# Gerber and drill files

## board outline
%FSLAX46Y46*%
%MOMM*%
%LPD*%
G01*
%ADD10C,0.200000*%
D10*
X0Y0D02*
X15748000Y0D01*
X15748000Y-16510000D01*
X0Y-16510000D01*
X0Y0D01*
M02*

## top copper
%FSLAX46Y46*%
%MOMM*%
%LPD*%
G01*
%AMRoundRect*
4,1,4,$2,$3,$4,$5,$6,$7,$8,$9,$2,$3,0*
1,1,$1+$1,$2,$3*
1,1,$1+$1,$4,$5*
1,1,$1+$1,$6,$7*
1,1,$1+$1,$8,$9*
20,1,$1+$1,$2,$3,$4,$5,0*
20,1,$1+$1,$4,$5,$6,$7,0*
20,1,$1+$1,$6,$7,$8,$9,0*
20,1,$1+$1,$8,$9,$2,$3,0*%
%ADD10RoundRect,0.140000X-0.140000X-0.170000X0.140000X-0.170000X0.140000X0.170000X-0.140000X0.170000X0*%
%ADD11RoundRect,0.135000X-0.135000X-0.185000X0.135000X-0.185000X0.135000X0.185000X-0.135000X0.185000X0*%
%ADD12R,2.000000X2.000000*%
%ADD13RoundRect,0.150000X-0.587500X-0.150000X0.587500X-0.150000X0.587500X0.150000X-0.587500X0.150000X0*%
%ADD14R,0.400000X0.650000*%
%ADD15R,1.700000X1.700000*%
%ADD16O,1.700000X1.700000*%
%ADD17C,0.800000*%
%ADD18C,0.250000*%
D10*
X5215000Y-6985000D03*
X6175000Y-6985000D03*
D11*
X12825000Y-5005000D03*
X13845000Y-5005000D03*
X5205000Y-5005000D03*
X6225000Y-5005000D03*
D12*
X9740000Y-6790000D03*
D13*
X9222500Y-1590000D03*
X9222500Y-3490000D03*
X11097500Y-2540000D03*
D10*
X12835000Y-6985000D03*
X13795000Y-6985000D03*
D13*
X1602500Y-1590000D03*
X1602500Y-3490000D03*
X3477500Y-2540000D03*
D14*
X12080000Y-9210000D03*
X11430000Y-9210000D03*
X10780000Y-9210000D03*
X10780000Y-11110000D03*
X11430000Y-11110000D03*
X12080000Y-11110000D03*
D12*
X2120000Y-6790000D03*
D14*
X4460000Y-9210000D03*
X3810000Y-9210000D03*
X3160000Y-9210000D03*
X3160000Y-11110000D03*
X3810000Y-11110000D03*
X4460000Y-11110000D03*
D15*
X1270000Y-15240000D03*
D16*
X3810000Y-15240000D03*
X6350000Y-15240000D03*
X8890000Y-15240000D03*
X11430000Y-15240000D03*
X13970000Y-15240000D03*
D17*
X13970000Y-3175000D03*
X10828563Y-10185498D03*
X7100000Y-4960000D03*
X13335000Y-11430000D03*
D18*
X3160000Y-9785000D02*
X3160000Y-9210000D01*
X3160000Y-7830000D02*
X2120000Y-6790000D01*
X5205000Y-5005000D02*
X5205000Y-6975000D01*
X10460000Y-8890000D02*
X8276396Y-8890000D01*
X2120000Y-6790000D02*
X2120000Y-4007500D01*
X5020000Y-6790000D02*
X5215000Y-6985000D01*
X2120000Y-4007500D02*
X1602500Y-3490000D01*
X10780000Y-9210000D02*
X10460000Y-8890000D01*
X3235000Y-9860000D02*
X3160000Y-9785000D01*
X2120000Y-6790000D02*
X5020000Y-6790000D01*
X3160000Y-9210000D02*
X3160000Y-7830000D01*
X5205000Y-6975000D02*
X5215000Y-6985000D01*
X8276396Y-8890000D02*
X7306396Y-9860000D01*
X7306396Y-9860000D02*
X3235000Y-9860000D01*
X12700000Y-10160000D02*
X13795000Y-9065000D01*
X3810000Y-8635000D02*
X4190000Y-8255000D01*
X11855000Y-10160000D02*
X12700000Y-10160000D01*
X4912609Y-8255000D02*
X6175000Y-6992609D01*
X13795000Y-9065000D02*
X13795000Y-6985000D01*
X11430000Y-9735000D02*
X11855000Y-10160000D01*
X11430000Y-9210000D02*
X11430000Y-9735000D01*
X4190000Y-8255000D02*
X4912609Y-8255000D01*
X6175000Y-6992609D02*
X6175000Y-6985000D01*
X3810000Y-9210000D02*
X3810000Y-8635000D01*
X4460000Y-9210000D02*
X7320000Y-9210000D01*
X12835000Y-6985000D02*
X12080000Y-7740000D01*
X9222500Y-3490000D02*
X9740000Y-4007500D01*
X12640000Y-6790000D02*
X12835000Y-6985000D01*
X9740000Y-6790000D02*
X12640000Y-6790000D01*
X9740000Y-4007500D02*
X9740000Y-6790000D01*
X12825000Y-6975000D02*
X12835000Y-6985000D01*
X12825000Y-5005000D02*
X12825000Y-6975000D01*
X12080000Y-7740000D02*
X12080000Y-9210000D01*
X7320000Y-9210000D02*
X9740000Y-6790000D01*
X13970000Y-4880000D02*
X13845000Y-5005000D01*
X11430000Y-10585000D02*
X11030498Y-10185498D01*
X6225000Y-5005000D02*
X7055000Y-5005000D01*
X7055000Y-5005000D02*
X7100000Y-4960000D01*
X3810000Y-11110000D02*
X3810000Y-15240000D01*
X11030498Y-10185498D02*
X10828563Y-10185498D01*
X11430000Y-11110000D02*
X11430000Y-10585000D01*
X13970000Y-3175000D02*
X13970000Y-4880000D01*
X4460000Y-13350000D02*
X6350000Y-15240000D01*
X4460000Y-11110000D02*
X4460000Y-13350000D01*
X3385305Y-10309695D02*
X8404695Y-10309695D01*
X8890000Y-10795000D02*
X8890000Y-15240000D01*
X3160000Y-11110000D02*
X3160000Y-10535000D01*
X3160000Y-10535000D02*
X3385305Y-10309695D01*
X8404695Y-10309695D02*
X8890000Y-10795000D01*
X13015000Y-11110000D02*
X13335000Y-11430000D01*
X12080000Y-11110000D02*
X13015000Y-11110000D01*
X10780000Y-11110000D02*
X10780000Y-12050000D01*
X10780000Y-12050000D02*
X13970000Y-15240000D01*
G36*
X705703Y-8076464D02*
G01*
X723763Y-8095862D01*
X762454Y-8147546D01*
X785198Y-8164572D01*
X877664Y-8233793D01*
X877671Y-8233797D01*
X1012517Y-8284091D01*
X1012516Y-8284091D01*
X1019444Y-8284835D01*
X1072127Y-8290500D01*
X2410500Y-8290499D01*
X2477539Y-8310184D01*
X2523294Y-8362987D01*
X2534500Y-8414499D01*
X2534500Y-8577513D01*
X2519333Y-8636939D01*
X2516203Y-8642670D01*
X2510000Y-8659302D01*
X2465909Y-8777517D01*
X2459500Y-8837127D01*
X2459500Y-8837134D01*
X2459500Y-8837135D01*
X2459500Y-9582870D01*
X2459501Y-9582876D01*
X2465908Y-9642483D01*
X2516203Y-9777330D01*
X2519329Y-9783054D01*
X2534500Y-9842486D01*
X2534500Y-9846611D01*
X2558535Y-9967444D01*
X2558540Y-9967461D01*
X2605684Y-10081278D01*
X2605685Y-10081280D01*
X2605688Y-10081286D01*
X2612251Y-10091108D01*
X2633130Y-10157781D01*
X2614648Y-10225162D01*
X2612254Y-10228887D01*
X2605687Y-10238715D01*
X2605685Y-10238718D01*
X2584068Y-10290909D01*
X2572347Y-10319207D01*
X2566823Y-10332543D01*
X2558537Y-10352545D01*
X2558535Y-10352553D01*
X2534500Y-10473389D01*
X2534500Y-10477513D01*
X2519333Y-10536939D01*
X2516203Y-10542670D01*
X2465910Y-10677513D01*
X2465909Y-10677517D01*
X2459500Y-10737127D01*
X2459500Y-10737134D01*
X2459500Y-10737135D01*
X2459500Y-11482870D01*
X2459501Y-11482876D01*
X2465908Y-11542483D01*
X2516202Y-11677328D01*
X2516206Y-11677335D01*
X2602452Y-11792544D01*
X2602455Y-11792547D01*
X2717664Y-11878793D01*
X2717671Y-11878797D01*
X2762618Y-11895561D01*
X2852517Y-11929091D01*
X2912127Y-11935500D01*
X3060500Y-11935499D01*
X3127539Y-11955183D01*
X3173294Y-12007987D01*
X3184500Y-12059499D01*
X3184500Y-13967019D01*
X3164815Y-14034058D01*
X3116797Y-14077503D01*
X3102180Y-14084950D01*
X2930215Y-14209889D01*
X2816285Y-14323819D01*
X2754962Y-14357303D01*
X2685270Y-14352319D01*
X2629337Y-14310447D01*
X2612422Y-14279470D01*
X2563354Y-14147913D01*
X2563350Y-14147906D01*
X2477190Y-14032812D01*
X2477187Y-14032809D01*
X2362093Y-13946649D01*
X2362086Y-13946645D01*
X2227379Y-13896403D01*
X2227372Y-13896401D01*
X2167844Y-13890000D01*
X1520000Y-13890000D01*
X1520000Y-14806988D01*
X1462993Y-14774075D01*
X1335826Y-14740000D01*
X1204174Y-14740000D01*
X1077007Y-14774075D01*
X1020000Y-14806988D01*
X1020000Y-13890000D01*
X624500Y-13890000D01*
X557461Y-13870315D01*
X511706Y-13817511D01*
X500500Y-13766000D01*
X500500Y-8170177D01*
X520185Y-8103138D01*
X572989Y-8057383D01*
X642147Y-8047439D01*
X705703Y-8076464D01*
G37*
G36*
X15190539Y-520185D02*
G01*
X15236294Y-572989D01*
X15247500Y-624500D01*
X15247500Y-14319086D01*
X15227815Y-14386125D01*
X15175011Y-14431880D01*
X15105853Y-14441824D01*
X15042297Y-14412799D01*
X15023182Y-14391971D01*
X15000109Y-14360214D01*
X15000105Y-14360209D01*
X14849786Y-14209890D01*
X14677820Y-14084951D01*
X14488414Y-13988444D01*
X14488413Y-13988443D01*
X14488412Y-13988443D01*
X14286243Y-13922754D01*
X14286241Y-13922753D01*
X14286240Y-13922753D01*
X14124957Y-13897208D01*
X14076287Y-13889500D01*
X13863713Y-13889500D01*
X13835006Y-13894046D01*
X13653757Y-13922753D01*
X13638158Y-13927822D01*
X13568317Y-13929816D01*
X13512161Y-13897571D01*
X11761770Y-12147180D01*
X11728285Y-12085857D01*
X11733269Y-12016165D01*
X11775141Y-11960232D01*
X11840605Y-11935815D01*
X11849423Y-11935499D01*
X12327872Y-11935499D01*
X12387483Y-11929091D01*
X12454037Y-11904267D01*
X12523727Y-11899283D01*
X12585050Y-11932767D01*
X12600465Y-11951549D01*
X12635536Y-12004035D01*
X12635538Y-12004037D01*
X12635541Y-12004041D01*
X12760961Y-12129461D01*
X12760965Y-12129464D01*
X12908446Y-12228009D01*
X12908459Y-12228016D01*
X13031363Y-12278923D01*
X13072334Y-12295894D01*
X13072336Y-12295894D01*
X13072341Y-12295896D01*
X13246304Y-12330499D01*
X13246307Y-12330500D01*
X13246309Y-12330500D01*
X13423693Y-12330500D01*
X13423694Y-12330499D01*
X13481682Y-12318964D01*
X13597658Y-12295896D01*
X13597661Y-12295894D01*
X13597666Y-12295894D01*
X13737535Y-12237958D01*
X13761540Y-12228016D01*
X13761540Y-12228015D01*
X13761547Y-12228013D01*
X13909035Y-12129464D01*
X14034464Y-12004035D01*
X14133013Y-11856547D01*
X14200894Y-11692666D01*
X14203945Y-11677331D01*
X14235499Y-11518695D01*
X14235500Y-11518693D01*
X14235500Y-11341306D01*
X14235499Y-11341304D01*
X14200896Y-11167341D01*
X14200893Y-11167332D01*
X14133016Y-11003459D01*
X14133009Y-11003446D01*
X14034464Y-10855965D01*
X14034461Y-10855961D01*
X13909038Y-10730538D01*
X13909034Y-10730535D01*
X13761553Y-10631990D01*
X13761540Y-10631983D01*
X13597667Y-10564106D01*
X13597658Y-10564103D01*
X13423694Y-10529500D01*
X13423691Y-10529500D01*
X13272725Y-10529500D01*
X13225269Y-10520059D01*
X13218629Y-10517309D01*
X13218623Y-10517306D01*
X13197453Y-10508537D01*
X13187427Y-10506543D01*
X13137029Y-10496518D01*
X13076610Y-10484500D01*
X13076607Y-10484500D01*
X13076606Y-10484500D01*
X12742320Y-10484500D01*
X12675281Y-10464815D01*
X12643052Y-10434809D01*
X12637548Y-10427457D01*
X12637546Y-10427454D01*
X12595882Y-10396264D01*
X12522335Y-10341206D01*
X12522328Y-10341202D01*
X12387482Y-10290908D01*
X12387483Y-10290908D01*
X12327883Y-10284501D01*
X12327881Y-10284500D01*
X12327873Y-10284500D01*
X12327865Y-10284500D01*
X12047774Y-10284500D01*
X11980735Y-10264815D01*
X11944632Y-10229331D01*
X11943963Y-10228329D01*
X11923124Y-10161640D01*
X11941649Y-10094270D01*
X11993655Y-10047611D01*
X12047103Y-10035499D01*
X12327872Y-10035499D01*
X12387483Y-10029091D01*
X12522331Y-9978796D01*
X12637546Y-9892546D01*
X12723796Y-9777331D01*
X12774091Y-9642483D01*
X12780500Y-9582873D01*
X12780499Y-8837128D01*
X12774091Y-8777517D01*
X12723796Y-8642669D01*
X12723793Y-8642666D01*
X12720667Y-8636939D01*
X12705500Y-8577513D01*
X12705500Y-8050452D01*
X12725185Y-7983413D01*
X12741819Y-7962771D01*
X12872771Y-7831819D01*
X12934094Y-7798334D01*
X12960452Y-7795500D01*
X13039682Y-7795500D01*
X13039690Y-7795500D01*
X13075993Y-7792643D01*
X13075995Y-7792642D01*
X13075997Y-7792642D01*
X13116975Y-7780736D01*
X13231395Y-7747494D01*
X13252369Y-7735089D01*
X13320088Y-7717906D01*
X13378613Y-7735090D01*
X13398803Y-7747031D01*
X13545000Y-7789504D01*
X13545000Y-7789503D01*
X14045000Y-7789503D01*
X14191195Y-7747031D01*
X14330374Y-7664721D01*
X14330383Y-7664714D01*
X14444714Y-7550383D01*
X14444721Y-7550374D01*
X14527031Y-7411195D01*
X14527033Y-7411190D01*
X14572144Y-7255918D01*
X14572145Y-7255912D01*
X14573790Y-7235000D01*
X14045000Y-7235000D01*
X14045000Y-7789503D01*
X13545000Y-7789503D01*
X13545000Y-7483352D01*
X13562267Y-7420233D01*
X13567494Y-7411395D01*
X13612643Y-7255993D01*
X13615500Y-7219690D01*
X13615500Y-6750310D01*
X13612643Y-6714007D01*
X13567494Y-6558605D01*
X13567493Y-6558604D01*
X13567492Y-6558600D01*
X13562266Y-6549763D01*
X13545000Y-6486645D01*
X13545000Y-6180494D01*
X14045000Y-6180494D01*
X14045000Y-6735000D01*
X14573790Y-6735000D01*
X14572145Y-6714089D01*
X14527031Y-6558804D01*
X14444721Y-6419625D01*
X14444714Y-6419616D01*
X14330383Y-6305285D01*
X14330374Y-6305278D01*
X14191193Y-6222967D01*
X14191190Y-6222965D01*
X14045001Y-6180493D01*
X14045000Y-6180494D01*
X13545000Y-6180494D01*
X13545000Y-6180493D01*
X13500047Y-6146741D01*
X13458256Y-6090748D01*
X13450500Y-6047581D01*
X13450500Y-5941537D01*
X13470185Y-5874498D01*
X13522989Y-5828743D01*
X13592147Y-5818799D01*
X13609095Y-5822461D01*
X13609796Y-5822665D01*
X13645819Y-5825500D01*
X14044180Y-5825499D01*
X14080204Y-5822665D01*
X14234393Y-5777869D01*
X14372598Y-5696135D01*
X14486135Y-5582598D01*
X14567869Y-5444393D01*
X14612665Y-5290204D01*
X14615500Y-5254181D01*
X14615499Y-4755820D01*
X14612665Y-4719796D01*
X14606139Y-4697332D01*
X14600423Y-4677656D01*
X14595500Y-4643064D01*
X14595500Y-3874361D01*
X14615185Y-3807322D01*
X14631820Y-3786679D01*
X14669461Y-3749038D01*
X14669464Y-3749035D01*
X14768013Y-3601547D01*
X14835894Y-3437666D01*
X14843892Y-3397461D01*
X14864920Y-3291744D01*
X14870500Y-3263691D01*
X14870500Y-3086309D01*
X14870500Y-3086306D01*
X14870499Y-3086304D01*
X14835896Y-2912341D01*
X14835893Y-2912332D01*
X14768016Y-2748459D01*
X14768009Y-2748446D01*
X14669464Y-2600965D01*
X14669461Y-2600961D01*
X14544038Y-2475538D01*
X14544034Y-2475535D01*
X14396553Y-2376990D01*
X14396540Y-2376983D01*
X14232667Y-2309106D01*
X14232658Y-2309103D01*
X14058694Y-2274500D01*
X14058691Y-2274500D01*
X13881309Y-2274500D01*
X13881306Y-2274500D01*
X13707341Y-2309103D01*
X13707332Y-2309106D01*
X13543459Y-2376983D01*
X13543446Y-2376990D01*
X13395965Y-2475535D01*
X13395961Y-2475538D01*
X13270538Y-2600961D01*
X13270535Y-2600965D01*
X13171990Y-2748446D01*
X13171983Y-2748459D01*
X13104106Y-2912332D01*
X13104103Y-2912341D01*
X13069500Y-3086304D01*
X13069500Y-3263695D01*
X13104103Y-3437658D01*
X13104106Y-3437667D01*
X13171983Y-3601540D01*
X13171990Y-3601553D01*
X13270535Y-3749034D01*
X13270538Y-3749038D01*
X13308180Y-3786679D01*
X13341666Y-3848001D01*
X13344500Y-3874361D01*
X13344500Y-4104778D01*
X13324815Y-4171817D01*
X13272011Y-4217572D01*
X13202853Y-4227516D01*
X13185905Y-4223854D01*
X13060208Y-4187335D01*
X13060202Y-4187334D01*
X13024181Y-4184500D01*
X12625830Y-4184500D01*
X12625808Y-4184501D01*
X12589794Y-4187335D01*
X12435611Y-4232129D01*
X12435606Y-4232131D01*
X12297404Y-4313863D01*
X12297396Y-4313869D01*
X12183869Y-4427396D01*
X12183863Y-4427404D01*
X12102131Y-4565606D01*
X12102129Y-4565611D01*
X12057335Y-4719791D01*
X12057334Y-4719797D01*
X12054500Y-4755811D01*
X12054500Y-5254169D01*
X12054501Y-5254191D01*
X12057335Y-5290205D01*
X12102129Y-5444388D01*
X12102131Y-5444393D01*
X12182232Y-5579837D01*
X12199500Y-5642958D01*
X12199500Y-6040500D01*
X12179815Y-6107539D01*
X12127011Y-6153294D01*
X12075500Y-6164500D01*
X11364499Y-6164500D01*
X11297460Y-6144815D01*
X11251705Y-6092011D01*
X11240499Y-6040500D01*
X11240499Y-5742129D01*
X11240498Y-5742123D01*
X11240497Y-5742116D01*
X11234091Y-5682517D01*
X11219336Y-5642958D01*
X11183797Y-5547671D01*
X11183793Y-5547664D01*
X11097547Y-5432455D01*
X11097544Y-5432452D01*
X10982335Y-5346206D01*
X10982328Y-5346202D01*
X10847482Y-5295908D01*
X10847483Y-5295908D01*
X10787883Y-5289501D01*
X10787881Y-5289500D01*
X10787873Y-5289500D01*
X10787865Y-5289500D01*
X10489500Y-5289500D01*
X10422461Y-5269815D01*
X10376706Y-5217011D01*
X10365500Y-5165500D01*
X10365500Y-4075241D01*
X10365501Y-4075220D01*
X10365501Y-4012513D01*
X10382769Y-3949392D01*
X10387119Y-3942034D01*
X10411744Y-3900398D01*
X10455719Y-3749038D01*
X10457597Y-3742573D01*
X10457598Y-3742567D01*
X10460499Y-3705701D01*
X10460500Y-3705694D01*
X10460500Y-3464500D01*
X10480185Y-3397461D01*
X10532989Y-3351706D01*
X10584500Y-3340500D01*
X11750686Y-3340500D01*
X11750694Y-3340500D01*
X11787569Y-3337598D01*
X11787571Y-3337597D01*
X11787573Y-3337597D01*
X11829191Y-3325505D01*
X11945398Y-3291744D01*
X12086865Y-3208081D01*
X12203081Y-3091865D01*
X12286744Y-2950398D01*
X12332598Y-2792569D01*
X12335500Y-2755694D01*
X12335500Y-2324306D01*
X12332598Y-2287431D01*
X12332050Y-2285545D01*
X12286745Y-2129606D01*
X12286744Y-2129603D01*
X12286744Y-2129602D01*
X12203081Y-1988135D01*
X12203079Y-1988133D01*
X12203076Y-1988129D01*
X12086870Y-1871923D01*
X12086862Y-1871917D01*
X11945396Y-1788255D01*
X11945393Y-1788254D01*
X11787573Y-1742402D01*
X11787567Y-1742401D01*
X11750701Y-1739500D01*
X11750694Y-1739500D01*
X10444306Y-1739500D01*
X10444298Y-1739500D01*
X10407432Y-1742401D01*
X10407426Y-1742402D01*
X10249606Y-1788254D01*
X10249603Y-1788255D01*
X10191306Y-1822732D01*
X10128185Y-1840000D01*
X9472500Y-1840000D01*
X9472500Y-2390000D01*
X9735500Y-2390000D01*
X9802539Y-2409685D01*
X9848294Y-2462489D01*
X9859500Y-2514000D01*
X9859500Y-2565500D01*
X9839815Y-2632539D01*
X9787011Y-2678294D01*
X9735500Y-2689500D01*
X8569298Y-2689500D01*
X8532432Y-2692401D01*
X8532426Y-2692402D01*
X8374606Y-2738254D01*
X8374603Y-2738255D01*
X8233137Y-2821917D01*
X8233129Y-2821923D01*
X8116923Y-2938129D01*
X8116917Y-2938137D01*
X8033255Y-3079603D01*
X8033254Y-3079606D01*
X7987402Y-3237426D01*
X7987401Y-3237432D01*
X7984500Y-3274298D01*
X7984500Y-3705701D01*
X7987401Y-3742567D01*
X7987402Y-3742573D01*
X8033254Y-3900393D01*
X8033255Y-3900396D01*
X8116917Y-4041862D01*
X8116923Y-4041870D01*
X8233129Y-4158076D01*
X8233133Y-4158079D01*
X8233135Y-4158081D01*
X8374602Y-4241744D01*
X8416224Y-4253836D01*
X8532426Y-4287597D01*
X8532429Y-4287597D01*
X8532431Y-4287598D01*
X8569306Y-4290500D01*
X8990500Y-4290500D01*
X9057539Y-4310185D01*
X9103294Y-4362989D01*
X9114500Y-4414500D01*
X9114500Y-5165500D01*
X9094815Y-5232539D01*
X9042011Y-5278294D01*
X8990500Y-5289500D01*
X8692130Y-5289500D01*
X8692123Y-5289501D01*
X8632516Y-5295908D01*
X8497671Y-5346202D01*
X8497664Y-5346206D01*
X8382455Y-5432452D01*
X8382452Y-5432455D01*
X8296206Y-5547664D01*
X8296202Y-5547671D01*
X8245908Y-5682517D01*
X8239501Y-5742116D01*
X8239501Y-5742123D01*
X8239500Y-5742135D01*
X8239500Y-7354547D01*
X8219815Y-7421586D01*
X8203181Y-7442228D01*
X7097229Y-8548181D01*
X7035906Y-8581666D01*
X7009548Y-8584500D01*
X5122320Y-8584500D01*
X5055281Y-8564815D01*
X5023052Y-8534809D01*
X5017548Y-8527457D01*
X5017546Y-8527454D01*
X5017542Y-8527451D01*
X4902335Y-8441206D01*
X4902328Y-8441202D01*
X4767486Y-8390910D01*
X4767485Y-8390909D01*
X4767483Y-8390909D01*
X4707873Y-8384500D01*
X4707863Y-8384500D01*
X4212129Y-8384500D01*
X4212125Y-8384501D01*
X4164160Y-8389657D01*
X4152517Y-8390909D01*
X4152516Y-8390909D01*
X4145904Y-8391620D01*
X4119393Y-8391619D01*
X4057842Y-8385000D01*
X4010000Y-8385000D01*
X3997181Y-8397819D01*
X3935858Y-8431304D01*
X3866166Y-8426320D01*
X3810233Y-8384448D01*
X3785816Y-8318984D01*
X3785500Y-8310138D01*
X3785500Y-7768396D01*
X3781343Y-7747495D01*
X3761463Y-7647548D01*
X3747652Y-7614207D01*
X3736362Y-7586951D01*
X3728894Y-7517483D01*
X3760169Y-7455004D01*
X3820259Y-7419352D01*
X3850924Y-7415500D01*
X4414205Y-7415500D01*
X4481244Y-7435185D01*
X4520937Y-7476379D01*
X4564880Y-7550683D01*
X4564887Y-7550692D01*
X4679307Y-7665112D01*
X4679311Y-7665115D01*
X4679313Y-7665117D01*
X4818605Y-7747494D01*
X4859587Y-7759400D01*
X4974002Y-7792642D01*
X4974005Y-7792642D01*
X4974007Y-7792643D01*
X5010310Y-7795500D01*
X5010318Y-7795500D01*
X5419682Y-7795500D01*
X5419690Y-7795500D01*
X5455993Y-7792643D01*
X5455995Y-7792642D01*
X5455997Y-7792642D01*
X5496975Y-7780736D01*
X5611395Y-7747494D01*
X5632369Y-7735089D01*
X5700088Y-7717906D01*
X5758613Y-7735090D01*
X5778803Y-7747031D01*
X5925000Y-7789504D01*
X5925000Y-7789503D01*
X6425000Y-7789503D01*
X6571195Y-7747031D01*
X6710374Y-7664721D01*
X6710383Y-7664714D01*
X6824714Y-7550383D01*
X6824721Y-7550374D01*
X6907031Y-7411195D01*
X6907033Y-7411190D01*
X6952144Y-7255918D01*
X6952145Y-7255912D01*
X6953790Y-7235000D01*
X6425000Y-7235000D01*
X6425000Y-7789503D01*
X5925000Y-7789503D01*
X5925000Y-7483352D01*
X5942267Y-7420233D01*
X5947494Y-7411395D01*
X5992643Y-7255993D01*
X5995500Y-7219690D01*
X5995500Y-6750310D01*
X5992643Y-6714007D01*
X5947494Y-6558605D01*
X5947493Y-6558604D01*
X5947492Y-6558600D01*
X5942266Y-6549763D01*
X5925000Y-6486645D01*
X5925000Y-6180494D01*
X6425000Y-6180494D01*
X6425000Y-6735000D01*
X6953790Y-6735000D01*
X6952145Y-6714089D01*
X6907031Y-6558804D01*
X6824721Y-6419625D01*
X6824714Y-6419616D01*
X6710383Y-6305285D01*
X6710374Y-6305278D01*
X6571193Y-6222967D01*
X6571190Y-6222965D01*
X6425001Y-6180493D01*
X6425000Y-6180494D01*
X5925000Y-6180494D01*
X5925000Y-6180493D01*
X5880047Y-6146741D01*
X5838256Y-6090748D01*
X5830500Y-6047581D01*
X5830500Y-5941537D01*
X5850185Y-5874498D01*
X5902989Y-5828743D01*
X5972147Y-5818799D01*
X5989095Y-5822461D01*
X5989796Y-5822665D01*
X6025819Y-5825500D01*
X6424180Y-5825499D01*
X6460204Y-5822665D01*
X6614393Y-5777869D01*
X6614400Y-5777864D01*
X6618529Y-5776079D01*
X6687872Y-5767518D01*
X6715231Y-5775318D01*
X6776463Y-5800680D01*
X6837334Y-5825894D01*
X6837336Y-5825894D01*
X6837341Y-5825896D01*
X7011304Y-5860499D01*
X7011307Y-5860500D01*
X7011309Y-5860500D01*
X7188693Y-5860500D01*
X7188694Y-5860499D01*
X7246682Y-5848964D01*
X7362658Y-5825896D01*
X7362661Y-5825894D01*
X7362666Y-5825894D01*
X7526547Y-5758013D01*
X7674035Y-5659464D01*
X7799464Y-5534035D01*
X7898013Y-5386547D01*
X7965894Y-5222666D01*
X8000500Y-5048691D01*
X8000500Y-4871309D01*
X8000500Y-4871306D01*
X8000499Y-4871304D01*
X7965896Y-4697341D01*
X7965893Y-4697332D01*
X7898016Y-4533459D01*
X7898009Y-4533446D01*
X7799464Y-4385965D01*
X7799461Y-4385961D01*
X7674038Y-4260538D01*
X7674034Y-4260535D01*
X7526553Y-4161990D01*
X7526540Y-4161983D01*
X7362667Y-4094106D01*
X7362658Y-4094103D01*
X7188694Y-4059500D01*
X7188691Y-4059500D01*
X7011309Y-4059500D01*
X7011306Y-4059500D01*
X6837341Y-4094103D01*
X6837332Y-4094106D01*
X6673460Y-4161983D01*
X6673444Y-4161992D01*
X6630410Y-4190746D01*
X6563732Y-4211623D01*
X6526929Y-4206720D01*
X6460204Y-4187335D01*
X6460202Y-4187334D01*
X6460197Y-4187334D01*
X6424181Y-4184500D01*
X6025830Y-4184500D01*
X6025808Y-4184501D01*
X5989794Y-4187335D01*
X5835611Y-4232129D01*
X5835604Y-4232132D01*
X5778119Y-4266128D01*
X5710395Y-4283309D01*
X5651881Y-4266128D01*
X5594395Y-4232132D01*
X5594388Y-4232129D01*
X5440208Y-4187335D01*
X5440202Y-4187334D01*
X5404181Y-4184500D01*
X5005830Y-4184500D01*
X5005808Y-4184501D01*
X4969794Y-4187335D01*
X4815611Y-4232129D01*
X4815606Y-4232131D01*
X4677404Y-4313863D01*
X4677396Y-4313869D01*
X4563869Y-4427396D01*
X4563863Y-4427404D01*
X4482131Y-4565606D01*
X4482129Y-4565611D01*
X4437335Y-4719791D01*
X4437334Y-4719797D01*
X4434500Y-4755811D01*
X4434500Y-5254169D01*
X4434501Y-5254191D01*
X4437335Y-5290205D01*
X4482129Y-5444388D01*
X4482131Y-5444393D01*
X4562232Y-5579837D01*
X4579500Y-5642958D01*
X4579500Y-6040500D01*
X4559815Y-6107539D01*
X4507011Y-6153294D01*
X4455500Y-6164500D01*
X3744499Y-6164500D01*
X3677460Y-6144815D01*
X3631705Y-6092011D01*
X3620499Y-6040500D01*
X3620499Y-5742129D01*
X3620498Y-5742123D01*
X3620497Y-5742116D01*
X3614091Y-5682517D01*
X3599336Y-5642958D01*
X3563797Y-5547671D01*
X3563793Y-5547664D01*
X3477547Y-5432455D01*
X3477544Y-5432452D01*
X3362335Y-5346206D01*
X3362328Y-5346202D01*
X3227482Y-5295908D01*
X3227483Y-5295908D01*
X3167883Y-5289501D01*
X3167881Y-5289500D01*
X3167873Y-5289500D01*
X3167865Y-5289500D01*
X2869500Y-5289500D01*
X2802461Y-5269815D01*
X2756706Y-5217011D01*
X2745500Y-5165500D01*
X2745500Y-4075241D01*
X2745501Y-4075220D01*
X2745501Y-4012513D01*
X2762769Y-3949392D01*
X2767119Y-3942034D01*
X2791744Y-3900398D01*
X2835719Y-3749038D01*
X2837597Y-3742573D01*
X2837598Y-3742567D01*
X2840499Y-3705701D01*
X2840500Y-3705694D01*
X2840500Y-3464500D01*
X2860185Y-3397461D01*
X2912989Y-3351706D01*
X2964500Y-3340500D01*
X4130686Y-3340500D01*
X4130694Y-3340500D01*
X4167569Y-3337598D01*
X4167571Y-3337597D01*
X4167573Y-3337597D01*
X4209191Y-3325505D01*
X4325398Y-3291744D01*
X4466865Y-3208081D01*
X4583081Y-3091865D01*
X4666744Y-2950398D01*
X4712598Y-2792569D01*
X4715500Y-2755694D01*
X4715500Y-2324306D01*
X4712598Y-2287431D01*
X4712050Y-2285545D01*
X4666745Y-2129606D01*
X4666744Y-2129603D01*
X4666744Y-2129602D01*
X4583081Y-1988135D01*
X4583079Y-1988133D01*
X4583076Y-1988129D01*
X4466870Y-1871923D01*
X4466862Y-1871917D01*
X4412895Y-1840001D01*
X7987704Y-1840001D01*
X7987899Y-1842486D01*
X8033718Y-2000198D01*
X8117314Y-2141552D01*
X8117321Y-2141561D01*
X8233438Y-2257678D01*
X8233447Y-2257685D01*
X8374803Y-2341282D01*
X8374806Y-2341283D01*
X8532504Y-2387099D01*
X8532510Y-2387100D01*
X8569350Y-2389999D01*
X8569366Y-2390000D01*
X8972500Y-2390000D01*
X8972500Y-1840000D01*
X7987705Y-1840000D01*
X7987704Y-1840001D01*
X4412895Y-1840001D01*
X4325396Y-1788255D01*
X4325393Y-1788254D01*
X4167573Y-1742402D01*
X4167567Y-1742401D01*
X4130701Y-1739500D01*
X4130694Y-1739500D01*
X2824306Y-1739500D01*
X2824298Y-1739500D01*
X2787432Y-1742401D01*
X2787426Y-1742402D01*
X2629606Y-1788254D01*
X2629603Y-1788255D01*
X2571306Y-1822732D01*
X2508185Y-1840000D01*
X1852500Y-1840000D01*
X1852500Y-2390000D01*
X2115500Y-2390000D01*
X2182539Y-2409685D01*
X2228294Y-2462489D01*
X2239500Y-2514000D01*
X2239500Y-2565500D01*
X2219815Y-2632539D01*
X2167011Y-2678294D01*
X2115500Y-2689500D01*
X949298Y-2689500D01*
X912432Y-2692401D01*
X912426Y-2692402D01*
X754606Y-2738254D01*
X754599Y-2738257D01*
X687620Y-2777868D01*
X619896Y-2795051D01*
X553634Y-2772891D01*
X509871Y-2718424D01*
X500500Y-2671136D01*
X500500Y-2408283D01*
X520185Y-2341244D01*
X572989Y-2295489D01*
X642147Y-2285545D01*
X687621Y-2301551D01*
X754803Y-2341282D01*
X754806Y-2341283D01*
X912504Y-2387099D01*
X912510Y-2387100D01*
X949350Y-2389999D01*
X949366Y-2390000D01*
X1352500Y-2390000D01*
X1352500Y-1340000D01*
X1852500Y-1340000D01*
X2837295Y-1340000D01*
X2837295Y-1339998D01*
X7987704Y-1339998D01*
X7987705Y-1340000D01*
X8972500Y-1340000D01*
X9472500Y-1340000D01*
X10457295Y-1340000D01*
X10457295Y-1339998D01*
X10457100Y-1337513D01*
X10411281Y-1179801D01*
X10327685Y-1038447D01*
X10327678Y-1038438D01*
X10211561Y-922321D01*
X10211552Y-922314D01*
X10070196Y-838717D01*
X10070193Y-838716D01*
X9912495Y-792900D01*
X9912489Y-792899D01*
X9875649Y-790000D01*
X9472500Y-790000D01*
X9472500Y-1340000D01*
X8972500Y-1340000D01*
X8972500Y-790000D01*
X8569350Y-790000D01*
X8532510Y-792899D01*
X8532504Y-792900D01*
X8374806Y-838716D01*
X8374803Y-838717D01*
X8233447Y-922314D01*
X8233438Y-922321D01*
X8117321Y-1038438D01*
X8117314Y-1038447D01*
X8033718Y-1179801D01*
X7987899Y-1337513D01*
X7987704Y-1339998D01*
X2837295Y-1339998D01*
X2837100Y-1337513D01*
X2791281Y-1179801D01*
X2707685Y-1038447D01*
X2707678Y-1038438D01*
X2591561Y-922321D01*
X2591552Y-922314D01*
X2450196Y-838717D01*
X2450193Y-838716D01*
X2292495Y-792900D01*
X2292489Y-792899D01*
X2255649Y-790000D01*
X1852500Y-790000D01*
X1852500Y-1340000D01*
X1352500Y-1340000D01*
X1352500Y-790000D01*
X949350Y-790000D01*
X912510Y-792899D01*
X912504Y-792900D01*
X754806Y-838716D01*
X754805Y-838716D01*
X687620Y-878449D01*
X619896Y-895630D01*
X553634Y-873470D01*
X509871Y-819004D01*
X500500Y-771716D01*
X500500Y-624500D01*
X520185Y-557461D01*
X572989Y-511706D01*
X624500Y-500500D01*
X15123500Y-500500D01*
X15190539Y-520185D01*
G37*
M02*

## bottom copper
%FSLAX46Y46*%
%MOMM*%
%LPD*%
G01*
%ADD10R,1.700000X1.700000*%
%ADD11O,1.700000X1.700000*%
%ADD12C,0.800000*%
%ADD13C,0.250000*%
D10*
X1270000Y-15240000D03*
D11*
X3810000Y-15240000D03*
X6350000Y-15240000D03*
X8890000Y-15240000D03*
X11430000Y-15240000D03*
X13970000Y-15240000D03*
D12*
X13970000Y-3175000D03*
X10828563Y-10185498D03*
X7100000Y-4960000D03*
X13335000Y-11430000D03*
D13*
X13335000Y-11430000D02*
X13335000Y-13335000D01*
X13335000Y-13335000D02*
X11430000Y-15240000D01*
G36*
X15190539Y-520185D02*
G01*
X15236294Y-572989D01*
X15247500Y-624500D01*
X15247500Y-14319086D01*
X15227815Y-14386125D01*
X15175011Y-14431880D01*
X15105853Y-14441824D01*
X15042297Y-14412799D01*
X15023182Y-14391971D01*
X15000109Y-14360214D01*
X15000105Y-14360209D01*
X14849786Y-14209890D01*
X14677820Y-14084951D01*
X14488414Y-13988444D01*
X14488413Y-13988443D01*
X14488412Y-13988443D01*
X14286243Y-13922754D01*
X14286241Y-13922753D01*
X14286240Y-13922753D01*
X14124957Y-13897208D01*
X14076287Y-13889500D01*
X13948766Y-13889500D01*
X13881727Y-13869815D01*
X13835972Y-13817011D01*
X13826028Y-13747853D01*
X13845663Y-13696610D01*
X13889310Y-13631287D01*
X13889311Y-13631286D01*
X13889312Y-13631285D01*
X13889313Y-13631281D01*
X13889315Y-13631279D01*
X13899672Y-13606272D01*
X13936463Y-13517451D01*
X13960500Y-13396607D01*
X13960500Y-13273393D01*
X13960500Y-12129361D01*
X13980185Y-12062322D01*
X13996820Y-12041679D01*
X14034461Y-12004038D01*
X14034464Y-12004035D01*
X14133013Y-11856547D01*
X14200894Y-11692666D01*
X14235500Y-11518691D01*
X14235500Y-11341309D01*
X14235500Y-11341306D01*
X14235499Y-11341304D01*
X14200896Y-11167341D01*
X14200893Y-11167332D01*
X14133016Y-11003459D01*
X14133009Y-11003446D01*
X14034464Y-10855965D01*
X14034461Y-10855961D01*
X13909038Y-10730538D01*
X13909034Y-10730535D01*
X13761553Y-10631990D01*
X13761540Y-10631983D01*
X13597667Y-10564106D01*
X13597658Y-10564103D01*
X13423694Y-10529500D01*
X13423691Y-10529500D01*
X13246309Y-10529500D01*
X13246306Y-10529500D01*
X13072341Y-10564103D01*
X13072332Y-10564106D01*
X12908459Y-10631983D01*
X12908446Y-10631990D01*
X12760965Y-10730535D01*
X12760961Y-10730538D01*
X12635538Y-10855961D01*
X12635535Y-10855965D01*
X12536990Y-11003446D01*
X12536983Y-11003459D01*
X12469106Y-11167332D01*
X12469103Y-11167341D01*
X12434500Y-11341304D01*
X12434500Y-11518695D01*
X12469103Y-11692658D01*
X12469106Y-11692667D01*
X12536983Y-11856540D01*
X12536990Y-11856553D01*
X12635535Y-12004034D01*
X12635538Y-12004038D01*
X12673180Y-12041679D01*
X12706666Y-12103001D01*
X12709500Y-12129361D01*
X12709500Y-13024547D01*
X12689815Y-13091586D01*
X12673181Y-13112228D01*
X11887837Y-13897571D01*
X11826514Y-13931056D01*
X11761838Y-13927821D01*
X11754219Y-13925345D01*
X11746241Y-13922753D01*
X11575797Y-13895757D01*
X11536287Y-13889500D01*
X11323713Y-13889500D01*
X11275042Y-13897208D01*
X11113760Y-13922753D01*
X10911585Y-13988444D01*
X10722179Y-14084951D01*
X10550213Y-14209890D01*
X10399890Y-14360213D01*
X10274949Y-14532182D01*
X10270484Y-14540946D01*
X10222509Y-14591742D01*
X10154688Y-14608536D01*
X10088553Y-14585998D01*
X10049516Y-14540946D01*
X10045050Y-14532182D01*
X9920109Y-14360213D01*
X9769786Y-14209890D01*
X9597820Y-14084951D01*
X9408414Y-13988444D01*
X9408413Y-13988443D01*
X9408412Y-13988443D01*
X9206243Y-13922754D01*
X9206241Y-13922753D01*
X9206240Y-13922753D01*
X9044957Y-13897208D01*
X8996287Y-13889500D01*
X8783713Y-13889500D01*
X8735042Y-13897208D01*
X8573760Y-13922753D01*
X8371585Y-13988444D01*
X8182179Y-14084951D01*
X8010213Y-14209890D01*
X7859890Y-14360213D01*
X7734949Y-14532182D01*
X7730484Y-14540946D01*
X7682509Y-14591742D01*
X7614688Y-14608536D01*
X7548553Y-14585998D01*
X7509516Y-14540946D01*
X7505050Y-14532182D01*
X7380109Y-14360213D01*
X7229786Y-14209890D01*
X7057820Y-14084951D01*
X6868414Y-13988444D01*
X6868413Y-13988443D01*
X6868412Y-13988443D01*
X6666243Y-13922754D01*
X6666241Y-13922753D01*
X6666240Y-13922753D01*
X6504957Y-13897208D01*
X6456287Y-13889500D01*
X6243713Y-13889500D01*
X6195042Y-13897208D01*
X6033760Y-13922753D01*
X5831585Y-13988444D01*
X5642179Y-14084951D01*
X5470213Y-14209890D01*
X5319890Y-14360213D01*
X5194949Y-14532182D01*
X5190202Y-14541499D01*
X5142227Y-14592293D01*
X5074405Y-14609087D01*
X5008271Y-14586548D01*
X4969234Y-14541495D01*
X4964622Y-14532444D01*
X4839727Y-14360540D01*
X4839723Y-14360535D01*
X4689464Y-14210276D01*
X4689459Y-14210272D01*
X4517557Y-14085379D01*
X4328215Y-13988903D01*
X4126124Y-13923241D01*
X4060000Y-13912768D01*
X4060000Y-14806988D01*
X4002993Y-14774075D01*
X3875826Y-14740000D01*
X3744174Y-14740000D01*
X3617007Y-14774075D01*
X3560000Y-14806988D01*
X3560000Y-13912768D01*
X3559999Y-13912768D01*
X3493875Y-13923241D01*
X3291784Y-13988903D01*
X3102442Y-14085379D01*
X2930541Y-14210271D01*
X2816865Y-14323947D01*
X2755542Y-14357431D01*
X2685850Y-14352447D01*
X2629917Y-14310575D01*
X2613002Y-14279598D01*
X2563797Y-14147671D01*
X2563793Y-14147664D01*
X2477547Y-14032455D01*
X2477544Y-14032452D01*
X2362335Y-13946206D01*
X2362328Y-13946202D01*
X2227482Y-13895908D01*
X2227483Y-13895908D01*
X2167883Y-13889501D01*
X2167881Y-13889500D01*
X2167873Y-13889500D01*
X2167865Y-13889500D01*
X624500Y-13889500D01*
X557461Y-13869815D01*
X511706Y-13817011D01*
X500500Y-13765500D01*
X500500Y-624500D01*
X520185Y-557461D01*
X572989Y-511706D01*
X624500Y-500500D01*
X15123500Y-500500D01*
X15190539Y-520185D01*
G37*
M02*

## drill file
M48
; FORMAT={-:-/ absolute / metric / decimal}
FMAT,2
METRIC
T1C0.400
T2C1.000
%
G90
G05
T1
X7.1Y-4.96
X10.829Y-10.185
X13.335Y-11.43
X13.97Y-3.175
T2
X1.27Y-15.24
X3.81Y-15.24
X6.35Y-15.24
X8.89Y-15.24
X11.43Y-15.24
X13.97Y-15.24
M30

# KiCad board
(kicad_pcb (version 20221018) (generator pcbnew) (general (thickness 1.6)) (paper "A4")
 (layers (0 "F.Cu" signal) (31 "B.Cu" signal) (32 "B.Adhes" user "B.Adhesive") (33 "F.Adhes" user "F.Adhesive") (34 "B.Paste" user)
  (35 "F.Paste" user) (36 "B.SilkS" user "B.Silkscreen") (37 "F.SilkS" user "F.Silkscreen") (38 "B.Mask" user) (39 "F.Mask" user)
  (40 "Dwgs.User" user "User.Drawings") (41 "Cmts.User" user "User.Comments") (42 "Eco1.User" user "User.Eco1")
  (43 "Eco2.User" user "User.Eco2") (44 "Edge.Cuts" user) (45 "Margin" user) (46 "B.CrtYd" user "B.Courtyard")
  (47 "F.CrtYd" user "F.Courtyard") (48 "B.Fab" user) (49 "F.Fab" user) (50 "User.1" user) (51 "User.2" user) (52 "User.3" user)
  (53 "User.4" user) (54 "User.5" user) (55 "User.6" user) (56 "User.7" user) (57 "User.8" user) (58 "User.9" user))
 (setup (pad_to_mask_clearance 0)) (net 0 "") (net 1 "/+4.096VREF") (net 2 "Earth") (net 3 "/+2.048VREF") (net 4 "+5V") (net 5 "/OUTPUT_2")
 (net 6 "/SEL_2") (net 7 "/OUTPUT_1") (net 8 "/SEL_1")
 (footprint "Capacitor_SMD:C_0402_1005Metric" (layer "F.Cu") (at 5.695 6.985)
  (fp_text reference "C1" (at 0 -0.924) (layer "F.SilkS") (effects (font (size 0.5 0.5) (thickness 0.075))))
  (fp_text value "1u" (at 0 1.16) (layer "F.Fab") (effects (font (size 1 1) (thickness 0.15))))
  (pad "1" smd roundrect (at -0.48 0) (size 0.56 0.62) (layers "F.Cu" "F.Paste" "F.Mask") (roundrect_rratio 0.25) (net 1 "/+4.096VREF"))
  (pad "2" smd roundrect (at 0.48 0) (size 0.56 0.62) (layers "F.Cu" "F.Paste" "F.Mask") (roundrect_rratio 0.25) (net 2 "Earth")))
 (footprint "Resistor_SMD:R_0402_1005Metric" (layer "F.Cu") (at 13.335 5.005)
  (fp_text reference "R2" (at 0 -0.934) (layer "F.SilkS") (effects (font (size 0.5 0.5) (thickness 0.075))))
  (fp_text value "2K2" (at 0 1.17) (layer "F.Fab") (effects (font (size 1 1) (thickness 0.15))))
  (pad "1" smd roundrect (at -0.51 0) (size 0.54 0.64) (layers "F.Cu" "F.Paste" "F.Mask") (roundrect_rratio 0.25) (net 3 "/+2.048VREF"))
  (pad "2" smd roundrect (at 0.51 0) (size 0.54 0.64) (layers "F.Cu" "F.Paste" "F.Mask") (roundrect_rratio 0.25) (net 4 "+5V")))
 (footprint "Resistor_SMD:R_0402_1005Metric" (layer "F.Cu") (at 5.715 5.005)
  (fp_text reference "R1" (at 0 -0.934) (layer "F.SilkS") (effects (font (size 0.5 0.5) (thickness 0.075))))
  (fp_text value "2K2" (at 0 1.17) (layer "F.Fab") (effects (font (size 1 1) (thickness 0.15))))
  (pad "1" smd roundrect (at -0.51 0) (size 0.54 0.64) (layers "F.Cu" "F.Paste" "F.Mask") (roundrect_rratio 0.25) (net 1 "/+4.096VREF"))
  (pad "2" smd roundrect (at 0.51 0) (size 0.54 0.64) (layers "F.Cu" "F.Paste" "F.Mask") (roundrect_rratio 0.25) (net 4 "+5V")))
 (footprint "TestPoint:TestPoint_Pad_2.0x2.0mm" (layer "F.Cu") (at 9.74 6.79)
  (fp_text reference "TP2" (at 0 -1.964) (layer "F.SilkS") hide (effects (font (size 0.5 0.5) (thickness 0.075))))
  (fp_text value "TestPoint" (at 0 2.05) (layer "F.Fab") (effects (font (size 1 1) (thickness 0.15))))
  (pad "1" smd rect (at 0 0) (size 2 2) (layers "F.Cu" "F.Mask") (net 3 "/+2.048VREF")))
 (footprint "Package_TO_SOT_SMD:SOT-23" (layer "F.Cu") (at 10.16 2.54)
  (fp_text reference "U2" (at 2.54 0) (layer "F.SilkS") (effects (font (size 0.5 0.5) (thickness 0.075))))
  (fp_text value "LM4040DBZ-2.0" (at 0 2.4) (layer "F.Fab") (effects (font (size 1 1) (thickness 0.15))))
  (pad "1" smd roundrect (at -0.9375 -0.95) (size 1.475 0.6) (layers "F.Cu" "F.Paste" "F.Mask") (roundrect_rratio 0.25) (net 2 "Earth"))
  (pad "2" smd roundrect (at -0.9375 0.95) (size 1.475 0.6) (layers "F.Cu" "F.Paste" "F.Mask") (roundrect_rratio 0.25) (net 3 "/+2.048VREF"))
  (pad "3" smd roundrect (at 0.9375 0) (size 1.475 0.6) (layers "F.Cu" "F.Paste" "F.Mask") (roundrect_rratio 0.25)))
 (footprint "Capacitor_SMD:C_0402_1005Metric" (layer "F.Cu") (at 13.315 6.985)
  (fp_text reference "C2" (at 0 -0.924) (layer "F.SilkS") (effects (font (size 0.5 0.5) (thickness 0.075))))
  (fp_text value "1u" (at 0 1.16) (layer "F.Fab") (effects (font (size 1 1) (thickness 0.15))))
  (pad "1" smd roundrect (at -0.48 0) (size 0.56 0.62) (layers "F.Cu" "F.Paste" "F.Mask") (roundrect_rratio 0.25) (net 3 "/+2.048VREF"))
  (pad "2" smd roundrect (at 0.48 0) (size 0.56 0.62) (layers "F.Cu" "F.Paste" "F.Mask") (roundrect_rratio 0.25) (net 2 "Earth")))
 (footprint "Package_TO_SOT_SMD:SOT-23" (layer "F.Cu") (at 2.54 2.54)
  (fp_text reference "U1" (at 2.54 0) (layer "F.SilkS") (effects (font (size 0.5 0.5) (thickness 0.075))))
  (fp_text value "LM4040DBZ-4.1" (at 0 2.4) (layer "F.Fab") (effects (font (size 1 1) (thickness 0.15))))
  (pad "1" smd roundrect (at -0.9375 -0.95) (size 1.475 0.6) (layers "F.Cu" "F.Paste" "F.Mask") (roundrect_rratio 0.25) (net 2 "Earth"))
  (pad "2" smd roundrect (at -0.9375 0.95) (size 1.475 0.6) (layers "F.Cu" "F.Paste" "F.Mask") (roundrect_rratio 0.25) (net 1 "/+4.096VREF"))
  (pad "3" smd roundrect (at 0.9375 0) (size 1.475 0.6) (layers "F.Cu" "F.Paste" "F.Mask") (roundrect_rratio 0.25)))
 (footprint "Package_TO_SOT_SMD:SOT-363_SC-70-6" (layer "F.Cu") (at 11.43 10.16 -90)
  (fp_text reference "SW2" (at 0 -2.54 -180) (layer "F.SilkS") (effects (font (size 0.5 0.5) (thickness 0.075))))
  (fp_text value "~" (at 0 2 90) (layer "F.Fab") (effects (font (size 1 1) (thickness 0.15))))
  (pad "1" smd rect (at -0.95 -0.65 270) (size 0.65 0.4) (layers "F.Cu" "F.Paste" "F.Mask") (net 3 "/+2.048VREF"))
  (pad "2" smd rect (at -0.95 0 270) (size 0.65 0.4) (layers "F.Cu" "F.Paste" "F.Mask") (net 2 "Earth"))
  (pad "3" smd rect (at -0.95 0.65 270) (size 0.65 0.4) (layers "F.Cu" "F.Paste" "F.Mask") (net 1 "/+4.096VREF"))
  (pad "4" smd rect (at 0.95 0.65 270) (size 0.65 0.4) (layers "F.Cu" "F.Paste" "F.Mask") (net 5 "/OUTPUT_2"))
  (pad "5" smd rect (at 0.95 0 270) (size 0.65 0.4) (layers "F.Cu" "F.Paste" "F.Mask") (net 4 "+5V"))
  (pad "6" smd rect (at 0.95 -0.65 270) (size 0.65 0.4) (layers "F.Cu" "F.Paste" "F.Mask") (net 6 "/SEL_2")))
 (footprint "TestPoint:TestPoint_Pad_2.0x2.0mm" (layer "F.Cu") (at 2.12 6.79)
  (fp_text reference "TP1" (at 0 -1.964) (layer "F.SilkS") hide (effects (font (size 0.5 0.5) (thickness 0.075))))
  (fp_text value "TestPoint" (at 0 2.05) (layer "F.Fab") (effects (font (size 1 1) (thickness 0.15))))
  (pad "1" smd rect (at 0 0) (size 2 2) (layers "F.Cu" "F.Mask") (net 1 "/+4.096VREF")))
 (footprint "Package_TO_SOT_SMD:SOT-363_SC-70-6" (layer "F.Cu") (at 3.81 10.16 -90)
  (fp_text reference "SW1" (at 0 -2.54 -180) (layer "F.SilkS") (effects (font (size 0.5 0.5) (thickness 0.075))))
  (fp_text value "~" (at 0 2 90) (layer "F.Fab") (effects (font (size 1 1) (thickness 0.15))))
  (pad "1" smd rect (at -0.95 -0.65 270) (size 0.65 0.4) (layers "F.Cu" "F.Paste" "F.Mask") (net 3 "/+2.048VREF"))
  (pad "2" smd rect (at -0.95 0 270) (size 0.65 0.4) (layers "F.Cu" "F.Paste" "F.Mask") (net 2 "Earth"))
  (pad "3" smd rect (at -0.95 0.65 270) (size 0.65 0.4) (layers "F.Cu" "F.Paste" "F.Mask") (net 1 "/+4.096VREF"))
  (pad "4" smd rect (at 0.95 0.65 270) (size 0.65 0.4) (layers "F.Cu" "F.Paste" "F.Mask") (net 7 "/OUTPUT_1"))
  (pad "5" smd rect (at 0.95 0 270) (size 0.65 0.4) (layers "F.Cu" "F.Paste" "F.Mask") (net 4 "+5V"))
  (pad "6" smd rect (at 0.95 -0.65 270) (size 0.65 0.4) (layers "F.Cu" "F.Paste" "F.Mask") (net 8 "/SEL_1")))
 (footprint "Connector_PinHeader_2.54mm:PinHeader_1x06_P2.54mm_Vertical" (layer "B.Cu") (at 1.27 15.24 -90)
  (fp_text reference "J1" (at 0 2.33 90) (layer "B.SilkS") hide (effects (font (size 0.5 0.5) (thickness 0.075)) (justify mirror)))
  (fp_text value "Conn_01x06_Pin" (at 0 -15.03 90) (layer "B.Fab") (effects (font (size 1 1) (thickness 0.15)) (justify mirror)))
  (pad "1" thru_hole rect (at 0 0 270) (size 1.7 1.7) (drill 1) (layers "*.Cu" "*.Mask") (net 2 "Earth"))
  (pad "2" thru_hole oval (at 0 -2.54 270) (size 1.7 1.7) (drill 1) (layers "*.Cu" "*.Mask") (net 4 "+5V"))
  (pad "3" thru_hole oval (at 0 -5.08 270) (size 1.7 1.7) (drill 1) (layers "*.Cu" "*.Mask") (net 8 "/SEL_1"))
  (pad "4" thru_hole oval (at 0 -7.62 270) (size 1.7 1.7) (drill 1) (layers "*.Cu" "*.Mask") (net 7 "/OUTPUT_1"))
  (pad "5" thru_hole oval (at 0 -10.16 270) (size 1.7 1.7) (drill 1) (layers "*.Cu" "*.Mask") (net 6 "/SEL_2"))
  (pad "6" thru_hole oval (at 0 -12.7 270) (size 1.7 1.7) (drill 1) (layers "*.Cu" "*.Mask") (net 5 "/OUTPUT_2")))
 (gr_rect (start 0 0) (end 15.748 16.51) (stroke (width 0.2) (type default)) (fill none) (layer "Edge.Cuts"))
 (segment (start 3.16 9.785) (end 3.16 9.21) (width 0.25) (layer "F.Cu") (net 1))
 (segment (start 3.16 7.83) (end 2.12 6.79) (width 0.25) (layer "F.Cu") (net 1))
 (segment (start 5.205 5.005) (end 5.205 6.975) (width 0.25) (layer "F.Cu") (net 1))
 (segment (start 10.46 8.89) (end 8.276396 8.89) (width 0.25) (layer "F.Cu") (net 1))
 (segment (start 2.12 6.79) (end 2.12 4.0075) (width 0.25) (layer "F.Cu") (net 1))
 (segment (start 5.02 6.79) (end 5.215 6.985) (width 0.25) (layer "F.Cu") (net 1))
 (segment (start 2.12 4.0075) (end 1.6025 3.49) (width 0.25) (layer "F.Cu") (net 1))
 (segment (start 10.78 9.21) (end 10.46 8.89) (width 0.25) (layer "F.Cu") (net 1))
 (segment (start 3.235 9.86) (end 3.16 9.785) (width 0.25) (layer "F.Cu") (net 1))
 (segment (start 2.12 6.79) (end 5.02 6.79) (width 0.25) (layer "F.Cu") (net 1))
 (segment (start 3.16 9.21) (end 3.16 7.83) (width 0.25) (layer "F.Cu") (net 1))
 (segment (start 5.205 6.975) (end 5.215 6.985) (width 0.25) (layer "F.Cu") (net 1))
 (segment (start 8.276396 8.89) (end 7.306396 9.86) (width 0.25) (layer "F.Cu") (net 1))
 (segment (start 7.306396 9.86) (end 3.235 9.86) (width 0.25) (layer "F.Cu") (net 1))
 (segment (start 12.7 10.16) (end 13.795 9.065) (width 0.25) (layer "F.Cu") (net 2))
 (segment (start 3.81 8.635) (end 4.19 8.255) (width 0.25) (layer "F.Cu") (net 2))
 (segment (start 11.855 10.16) (end 12.7 10.16) (width 0.25) (layer "F.Cu") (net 2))
 (segment (start 4.912609 8.255) (end 6.175 6.992609) (width 0.25) (layer "F.Cu") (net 2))
 (segment (start 13.795 9.065) (end 13.795 6.985) (width 0.25) (layer "F.Cu") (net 2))
 (segment (start 11.43 9.735) (end 11.855 10.16) (width 0.25) (layer "F.Cu") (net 2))
 (segment (start 11.43 9.21) (end 11.43 9.735) (width 0.25) (layer "F.Cu") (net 2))
 (segment (start 4.19 8.255) (end 4.912609 8.255) (width 0.25) (layer "F.Cu") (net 2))
 (segment (start 6.175 6.992609) (end 6.175 6.985) (width 0.25) (layer "F.Cu") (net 2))
 (segment (start 3.81 9.21) (end 3.81 8.635) (width 0.25) (layer "F.Cu") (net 2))
 (segment (start 4.46 9.21) (end 7.32 9.21) (width 0.25) (layer "F.Cu") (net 3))
 (segment (start 12.835 6.985) (end 12.08 7.74) (width 0.25) (layer "F.Cu") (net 3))
 (segment (start 9.2225 3.49) (end 9.74 4.0075) (width 0.25) (layer "F.Cu") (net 3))
 (segment (start 12.64 6.79) (end 12.835 6.985) (width 0.25) (layer "F.Cu") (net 3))
 (segment (start 9.74 6.79) (end 12.64 6.79) (width 0.25) (layer "F.Cu") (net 3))
 (segment (start 9.74 4.0075) (end 9.74 6.79) (width 0.25) (layer "F.Cu") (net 3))
 (segment (start 12.825 6.975) (end 12.835 6.985) (width 0.25) (layer "F.Cu") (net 3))
 (segment (start 12.825 5.005) (end 12.825 6.975) (width 0.25) (layer "F.Cu") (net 3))
 (segment (start 12.08 7.74) (end 12.08 9.21) (width 0.25) (layer "F.Cu") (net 3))
 (segment (start 7.32 9.21) (end 9.74 6.79) (width 0.25) (layer "F.Cu") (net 3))
 (segment (start 13.97 4.88) (end 13.845 5.005) (width 0.25) (layer "F.Cu") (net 4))
 (segment (start 11.43 10.585) (end 11.030498 10.185498) (width 0.25) (layer "F.Cu") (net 4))
 (segment (start 6.225 5.005) (end 7.055 5.005) (width 0.25) (layer "F.Cu") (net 4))
 (segment (start 7.055 5.005) (end 7.1 4.96) (width 0.25) (layer "F.Cu") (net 4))
 (segment (start 3.81 11.11) (end 3.81 15.24) (width 0.25) (layer "F.Cu") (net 4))
 (segment (start 11.030498 10.185498) (end 10.828563 10.185498) (width 0.25) (layer "F.Cu") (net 4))
 (segment (start 11.43 11.11) (end 11.43 10.585) (width 0.25) (layer "F.Cu") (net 4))
 (segment (start 13.97 3.175) (end 13.97 4.88) (width 0.25) (layer "F.Cu") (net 4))
 (via (at 13.97 3.175) (size 0.8) (drill 0.4) (layers "F.Cu" "B.Cu") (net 4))
 (via (at 10.828563 10.185498) (size 0.8) (drill 0.4) (layers "F.Cu" "B.Cu") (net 4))
 (via (at 7.1 4.96) (size 0.8) (drill 0.4) (layers "F.Cu" "B.Cu") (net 4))
 (segment (start 4.46 13.35) (end 6.35 15.24) (width 0.25) (layer "F.Cu") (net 8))
 (segment (start 4.46 11.11) (end 4.46 13.35) (width 0.25) (layer "F.Cu") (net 8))
 (segment (start 3.385305 10.309695) (end 8.404695 10.309695) (width 0.25) (layer "F.Cu") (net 7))
 (segment (start 8.89 10.795) (end 8.89 15.24) (width 0.25) (layer "F.Cu") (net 7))
 (segment (start 3.16 11.11) (end 3.16 10.535) (width 0.25) (layer "F.Cu") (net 7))
 (segment (start 3.16 10.535) (end 3.385305 10.309695) (width 0.25) (layer "F.Cu") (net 7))
 (segment (start 8.404695 10.309695) (end 8.89 10.795) (width 0.25) (layer "F.Cu") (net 7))
 (segment (start 13.015 11.11) (end 13.335 11.43) (width 0.25) (layer "F.Cu") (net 6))
 (segment (start 12.08 11.11) (end 13.015 11.11) (width 0.25) (layer "F.Cu") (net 6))
 (via (at 13.335 11.43) (size 0.8) (drill 0.4) (layers "F.Cu" "B.Cu") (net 6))
 (segment (start 13.335 11.43) (end 13.335 13.335) (width 0.25) (layer "B.Cu") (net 6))
 (segment (start 13.335 13.335) (end 11.43 15.24) (width 0.25) (layer "B.Cu") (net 6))
 (segment (start 10.78 11.11) (end 10.78 12.05) (width 0.25) (layer "F.Cu") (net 5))
 (segment (start 10.78 12.05) (end 13.97 15.24) (width 0.25) (layer "F.Cu") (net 5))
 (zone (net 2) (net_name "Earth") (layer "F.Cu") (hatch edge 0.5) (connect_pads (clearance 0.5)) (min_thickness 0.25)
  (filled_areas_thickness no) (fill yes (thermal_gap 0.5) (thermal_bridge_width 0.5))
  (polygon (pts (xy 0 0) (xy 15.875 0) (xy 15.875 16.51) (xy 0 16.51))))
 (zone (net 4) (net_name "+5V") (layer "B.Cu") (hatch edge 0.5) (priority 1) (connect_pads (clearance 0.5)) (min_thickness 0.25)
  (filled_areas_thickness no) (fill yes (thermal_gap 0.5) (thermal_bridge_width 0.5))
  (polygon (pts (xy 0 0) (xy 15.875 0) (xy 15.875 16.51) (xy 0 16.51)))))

